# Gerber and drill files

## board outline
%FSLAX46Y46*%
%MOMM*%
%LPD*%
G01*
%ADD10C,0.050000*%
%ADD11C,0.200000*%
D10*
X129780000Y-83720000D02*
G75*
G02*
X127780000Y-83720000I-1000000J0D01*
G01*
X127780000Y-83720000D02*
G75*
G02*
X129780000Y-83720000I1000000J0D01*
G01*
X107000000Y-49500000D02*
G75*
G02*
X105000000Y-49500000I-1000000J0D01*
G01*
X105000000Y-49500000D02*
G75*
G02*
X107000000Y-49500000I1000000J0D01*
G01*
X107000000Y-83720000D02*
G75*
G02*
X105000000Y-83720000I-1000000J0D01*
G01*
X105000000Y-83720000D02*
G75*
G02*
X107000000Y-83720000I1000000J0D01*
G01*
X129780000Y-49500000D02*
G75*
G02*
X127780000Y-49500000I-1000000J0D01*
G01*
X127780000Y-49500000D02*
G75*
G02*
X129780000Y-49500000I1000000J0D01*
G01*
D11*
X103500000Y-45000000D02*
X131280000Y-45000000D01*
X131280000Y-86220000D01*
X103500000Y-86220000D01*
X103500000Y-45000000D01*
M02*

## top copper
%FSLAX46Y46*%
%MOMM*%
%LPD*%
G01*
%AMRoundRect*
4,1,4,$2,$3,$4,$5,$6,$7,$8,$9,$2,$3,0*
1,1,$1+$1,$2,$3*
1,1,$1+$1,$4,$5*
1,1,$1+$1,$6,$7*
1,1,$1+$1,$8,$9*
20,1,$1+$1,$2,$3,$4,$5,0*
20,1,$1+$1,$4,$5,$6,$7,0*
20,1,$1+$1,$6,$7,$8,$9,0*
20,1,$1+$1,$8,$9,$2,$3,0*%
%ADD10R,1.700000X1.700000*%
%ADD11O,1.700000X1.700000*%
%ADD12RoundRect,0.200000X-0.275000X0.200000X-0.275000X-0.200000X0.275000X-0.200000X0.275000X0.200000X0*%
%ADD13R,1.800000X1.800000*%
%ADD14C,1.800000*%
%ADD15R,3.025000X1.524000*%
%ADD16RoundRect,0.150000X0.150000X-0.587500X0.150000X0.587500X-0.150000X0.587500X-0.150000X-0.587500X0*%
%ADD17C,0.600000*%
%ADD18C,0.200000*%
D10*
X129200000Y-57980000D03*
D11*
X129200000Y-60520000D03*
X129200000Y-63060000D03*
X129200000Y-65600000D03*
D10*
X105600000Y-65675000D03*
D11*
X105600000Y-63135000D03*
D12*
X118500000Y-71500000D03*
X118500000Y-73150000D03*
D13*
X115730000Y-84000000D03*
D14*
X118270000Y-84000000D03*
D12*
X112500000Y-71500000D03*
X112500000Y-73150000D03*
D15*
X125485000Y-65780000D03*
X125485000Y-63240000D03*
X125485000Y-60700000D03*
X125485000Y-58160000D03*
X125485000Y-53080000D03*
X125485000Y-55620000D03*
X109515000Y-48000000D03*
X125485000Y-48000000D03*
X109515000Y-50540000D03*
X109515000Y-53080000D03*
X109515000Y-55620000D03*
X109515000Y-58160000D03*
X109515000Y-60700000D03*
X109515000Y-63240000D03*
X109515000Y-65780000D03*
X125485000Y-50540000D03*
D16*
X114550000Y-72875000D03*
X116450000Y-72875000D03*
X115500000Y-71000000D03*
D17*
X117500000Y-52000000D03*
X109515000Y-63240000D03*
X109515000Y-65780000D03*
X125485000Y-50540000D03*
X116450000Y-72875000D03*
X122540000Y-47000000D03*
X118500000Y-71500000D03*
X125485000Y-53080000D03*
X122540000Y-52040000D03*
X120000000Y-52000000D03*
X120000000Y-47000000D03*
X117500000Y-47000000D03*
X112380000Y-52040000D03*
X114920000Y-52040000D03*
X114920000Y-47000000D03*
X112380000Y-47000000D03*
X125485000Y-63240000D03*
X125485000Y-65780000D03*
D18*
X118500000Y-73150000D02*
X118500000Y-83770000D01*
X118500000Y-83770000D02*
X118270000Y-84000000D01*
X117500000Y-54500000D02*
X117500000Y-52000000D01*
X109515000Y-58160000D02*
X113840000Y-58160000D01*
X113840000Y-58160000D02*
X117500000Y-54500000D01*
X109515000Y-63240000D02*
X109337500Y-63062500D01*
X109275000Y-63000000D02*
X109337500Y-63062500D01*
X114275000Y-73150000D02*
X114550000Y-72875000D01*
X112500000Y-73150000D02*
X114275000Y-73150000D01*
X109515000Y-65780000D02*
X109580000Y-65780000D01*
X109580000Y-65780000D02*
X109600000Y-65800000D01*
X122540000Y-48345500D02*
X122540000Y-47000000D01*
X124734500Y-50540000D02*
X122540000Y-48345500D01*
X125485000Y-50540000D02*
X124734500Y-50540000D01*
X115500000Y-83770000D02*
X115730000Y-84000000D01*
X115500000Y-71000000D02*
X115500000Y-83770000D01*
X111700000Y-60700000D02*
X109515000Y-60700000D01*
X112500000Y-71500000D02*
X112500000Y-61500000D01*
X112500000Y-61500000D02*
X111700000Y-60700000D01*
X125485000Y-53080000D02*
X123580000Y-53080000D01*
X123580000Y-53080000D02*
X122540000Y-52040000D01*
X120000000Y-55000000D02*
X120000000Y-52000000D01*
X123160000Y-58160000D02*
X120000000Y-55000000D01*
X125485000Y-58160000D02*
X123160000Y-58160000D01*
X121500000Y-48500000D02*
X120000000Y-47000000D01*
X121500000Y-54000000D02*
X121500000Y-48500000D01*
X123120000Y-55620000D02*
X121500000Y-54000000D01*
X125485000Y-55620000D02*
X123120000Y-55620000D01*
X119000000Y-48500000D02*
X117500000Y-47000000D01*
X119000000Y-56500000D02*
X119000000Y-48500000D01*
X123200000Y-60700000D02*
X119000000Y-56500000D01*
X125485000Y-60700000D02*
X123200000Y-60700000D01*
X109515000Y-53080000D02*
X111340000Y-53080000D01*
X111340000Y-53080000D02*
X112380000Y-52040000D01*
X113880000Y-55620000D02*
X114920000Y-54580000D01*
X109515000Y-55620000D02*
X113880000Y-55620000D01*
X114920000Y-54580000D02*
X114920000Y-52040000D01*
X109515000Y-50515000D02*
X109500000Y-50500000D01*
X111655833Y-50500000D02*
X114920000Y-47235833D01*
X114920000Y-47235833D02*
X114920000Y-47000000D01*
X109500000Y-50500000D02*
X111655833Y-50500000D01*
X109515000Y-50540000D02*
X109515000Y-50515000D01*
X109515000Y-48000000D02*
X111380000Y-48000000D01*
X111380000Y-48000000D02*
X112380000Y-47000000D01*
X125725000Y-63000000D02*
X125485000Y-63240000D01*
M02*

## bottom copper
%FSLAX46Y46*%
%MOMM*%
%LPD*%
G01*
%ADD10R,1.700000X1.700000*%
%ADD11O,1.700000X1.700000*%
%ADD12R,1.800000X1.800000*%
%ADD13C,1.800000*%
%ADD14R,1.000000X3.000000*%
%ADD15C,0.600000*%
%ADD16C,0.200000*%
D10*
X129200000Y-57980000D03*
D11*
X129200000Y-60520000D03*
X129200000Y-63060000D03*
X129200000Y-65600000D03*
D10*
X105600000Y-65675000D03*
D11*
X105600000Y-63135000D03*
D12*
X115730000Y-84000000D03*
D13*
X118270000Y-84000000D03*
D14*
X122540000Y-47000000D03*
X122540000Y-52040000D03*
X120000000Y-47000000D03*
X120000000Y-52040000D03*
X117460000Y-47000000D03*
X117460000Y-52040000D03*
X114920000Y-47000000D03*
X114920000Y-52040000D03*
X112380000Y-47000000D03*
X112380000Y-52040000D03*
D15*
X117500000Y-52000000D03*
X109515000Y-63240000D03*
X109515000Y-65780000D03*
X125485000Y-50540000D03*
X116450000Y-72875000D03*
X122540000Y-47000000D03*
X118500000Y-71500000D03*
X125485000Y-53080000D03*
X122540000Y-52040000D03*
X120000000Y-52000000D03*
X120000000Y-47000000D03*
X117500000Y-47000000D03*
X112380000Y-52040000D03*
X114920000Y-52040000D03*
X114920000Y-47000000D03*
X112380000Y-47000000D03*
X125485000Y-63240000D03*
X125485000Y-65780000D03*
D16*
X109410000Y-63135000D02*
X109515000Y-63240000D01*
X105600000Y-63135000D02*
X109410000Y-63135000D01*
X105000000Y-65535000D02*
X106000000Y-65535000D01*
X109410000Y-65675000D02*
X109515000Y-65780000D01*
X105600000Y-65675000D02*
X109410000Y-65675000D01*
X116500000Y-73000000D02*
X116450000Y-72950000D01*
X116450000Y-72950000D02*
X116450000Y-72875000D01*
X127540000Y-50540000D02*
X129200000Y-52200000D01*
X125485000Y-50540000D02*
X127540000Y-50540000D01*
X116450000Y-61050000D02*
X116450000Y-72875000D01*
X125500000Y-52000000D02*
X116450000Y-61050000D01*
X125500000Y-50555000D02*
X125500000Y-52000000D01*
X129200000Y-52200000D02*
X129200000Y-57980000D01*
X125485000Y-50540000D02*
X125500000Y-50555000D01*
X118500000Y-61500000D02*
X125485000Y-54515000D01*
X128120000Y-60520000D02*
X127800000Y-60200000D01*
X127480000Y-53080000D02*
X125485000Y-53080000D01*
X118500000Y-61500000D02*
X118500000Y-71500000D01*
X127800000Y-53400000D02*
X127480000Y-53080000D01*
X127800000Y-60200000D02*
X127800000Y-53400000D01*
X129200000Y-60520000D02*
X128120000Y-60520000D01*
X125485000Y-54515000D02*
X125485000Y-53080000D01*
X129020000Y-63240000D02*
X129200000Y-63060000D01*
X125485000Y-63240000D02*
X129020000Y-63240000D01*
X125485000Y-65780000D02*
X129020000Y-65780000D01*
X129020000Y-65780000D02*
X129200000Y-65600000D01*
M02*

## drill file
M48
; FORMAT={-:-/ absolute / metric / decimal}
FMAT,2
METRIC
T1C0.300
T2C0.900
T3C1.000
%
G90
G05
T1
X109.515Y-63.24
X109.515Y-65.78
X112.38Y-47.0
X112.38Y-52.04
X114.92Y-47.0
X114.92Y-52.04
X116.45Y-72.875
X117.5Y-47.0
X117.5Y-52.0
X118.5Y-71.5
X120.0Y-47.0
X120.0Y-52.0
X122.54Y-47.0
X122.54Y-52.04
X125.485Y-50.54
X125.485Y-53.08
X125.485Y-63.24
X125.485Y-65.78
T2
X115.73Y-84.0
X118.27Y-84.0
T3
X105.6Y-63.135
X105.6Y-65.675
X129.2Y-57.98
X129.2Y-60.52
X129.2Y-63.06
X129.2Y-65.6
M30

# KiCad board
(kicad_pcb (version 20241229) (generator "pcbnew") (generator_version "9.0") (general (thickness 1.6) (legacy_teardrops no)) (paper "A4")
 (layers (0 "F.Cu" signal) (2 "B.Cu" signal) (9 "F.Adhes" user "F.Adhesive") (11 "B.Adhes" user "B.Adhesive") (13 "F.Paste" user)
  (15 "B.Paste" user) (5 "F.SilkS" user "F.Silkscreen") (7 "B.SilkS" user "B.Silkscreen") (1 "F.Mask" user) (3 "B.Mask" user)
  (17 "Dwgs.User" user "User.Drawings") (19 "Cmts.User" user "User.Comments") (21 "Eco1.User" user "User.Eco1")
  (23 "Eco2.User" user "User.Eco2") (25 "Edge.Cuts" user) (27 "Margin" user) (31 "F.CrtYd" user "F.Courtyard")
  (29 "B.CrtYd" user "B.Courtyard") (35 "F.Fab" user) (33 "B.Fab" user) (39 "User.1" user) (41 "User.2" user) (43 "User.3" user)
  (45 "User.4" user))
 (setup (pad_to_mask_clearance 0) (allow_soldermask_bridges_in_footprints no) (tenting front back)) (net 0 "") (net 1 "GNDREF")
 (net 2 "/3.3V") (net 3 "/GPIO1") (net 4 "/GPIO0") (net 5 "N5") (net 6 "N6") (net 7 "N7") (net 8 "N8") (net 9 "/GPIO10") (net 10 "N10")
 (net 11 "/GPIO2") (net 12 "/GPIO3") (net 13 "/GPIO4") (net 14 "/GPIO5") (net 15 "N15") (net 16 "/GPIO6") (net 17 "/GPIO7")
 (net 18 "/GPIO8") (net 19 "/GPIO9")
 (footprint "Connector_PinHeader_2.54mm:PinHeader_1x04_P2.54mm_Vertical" (layer "F.Cu") (at 129.2 57.98)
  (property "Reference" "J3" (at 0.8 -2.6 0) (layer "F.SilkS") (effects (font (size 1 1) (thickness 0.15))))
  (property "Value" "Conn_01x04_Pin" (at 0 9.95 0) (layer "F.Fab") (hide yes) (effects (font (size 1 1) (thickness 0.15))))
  (pad "1" thru_hole rect (at 0 0) (size 1.7 1.7) (drill 1) (layers "*.Cu" "*.Mask") (remove_unused_layers no) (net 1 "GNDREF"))
  (pad "2" thru_hole oval (at 0 2.54) (size 1.7 1.7) (drill 1) (layers "*.Cu" "*.Mask") (remove_unused_layers no) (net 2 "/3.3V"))
  (pad "3" thru_hole oval (at 0 5.08) (size 1.7 1.7) (drill 1) (layers "*.Cu" "*.Mask") (remove_unused_layers no) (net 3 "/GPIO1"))
  (pad "4" thru_hole oval (at 0 7.62) (size 1.7 1.7) (drill 1) (layers "*.Cu" "*.Mask") (remove_unused_layers no) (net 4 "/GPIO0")))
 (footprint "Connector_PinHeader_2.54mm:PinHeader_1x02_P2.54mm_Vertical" (layer "F.Cu") (at 105.6 65.675 180)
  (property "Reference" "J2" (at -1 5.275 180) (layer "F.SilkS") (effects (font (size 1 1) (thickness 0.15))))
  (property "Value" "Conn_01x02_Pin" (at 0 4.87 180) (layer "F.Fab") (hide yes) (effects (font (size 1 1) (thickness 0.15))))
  (pad "1" thru_hole rect (at 0 0 180) (size 1.7 1.7) (drill 1) (layers "*.Cu" "*.Mask") (remove_unused_layers no) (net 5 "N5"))
  (pad "2" thru_hole oval (at 0 2.54 180) (size 1.7 1.7) (drill 1) (layers "*.Cu" "*.Mask") (remove_unused_layers no) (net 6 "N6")))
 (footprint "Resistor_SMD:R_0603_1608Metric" (layer "F.Cu") (at 118.5 72.325 -90)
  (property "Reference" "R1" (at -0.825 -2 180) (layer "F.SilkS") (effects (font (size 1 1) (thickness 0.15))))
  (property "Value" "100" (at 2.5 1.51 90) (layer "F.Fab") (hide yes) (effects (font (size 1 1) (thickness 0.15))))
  (pad "1" smd roundrect (at -0.825 0 270) (size 0.8 0.95) (layers "F.Cu" "F.Mask" "F.Paste") (roundrect_rratio 0.25) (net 2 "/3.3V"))
  (pad "2" smd roundrect (at 0.825 0 270) (size 0.8 0.95) (layers "F.Cu" "F.Mask" "F.Paste") (roundrect_rratio 0.25) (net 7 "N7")))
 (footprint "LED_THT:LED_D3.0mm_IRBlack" (layer "F.Cu") (at 115.73 84)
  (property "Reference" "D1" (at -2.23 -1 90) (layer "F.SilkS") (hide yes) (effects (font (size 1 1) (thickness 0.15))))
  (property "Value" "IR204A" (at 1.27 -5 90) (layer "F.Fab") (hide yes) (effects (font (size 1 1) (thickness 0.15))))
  (pad "1" thru_hole rect (at 0 0) (size 1.8 1.8) (drill 0.9) (layers "*.Cu" "*.Mask") (remove_unused_layers no) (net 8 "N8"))
  (pad "2" thru_hole circle (at 2.54 0) (size 1.8 1.8) (drill 0.9) (layers "*.Cu" "*.Mask") (remove_unused_layers no) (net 7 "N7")))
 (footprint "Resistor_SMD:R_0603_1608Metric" (layer "F.Cu") (at 112.5 72.325 -90)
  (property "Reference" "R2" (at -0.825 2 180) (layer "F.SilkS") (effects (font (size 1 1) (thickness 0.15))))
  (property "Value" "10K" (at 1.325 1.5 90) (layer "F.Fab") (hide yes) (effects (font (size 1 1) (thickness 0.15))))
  (pad "1" smd roundrect (at -0.825 0 270) (size 0.8 0.95) (layers "F.Cu" "F.Mask" "F.Paste") (roundrect_rratio 0.25) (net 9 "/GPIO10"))
  (pad "2" smd roundrect (at 0.825 0 270) (size 0.8 0.95) (layers "F.Cu" "F.Mask" "F.Paste") (roundrect_rratio 0.25) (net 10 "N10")))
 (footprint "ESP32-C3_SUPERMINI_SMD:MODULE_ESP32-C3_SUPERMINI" (layer "F.Cu") (at 117.5 57.9)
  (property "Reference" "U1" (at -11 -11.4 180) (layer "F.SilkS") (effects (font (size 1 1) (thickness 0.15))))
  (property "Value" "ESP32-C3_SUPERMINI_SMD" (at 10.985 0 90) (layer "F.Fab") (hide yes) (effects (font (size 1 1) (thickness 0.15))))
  (pad "0" smd rect (at 7.985 7.88) (size 3.025 1.524) (layers "F.Cu" "F.Mask" "F.Paste") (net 4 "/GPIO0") (solder_mask_margin 0.102))
  (pad "1" smd rect (at 7.985 5.34) (size 3.025 1.524) (layers "F.Cu" "F.Mask" "F.Paste") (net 3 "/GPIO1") (solder_mask_margin 0.102))
  (pad "2" smd rect (at 7.985 2.8) (size 3.025 1.524) (layers "F.Cu" "F.Mask" "F.Paste") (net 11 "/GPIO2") (solder_mask_margin 0.102))
  (pad "3" smd rect (at 7.985 0.26) (size 3.025 1.524) (layers "F.Cu" "F.Mask" "F.Paste") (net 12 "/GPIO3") (solder_mask_margin 0.102))
  (pad "3.3" smd rect (at 7.985 -4.82) (size 3.025 1.524) (layers "F.Cu" "F.Mask" "F.Paste") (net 2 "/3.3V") (solder_mask_margin 0.102))
  (pad "4" smd rect (at 7.985 -2.28) (size 3.025 1.524) (layers "F.Cu" "F.Mask" "F.Paste") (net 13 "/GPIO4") (solder_mask_margin 0.102))
  (pad "5" smd rect (at -7.985 -9.9) (size 3.025 1.524) (layers "F.Cu" "F.Mask" "F.Paste") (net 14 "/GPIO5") (solder_mask_margin 0.102))
  (pad "5V" smd rect (at 7.985 -9.9) (size 3.025 1.524) (layers "F.Cu" "F.Mask" "F.Paste") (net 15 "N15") (solder_mask_margin 0.102))
  (pad "6" smd rect (at -7.985 -7.36) (size 3.025 1.524) (layers "F.Cu" "F.Mask" "F.Paste") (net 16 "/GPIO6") (solder_mask_margin 0.102))
  (pad "7" smd rect (at -7.985 -4.82) (size 3.025 1.524) (layers "F.Cu" "F.Mask" "F.Paste") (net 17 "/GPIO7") (solder_mask_margin 0.102))
  (pad "8" smd rect (at -7.985 -2.28) (size 3.025 1.524) (layers "F.Cu" "F.Mask" "F.Paste") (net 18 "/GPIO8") (solder_mask_margin 0.102))
  (pad "9" smd rect (at -7.985 0.26) (size 3.025 1.524) (layers "F.Cu" "F.Mask" "F.Paste") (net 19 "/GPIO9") (solder_mask_margin 0.102))
  (pad "10" smd rect (at -7.985 2.8) (size 3.025 1.524) (layers "F.Cu" "F.Mask" "F.Paste") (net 9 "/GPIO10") (solder_mask_margin 0.102))
  (pad "20" smd rect (at -7.985 5.34) (size 3.025 1.524) (layers "F.Cu" "F.Mask" "F.Paste") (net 6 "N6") (solder_mask_margin 0.102))
  (pad "21" smd rect (at -7.985 7.88) (size 3.025 1.524) (layers "F.Cu" "F.Mask" "F.Paste") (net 5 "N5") (solder_mask_margin 0.102))
  (pad "G" smd rect (at 7.985 -7.36) (size 3.025 1.524) (layers "F.Cu" "F.Mask" "F.Paste") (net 1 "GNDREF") (solder_mask_margin 0.102)))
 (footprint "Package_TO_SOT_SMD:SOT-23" (layer "F.Cu") (at 115.5 71.9375 90)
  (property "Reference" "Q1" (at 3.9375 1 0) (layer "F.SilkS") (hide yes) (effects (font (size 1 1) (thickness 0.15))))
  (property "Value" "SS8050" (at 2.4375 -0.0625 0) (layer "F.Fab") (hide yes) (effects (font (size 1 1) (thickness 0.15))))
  (pad "1" smd roundrect (at -0.9375 -0.95 90) (size 1.475 0.6) (layers "F.Cu" "F.Mask" "F.Paste") (roundrect_rratio 0.25) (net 10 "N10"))
  (pad "2" smd roundrect (at -0.9375 0.95 90) (size 1.475 0.6) (layers "F.Cu" "F.Mask" "F.Paste") (roundrect_rratio 0.25) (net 1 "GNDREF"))
  (pad "3" smd roundrect (at 0.9375 0 90) (size 1.475 0.6) (layers "F.Cu" "F.Mask" "F.Paste") (roundrect_rratio 0.25) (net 8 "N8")))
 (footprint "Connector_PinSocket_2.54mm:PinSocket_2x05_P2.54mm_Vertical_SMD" (layer "B.Cu") (at 117.46 49.52 90)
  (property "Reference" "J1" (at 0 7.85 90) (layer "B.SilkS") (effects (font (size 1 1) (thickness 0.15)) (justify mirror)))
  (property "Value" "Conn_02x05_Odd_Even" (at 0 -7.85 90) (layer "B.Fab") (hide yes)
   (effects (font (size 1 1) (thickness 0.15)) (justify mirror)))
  (pad "1" smd rect (at 2.52 5.08 90) (size 3 1) (layers "B.Cu" "B.Mask" "B.Paste") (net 1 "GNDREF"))
  (pad "2" smd rect (at -2.52 5.08 90) (size 3 1) (layers "B.Cu" "B.Mask" "B.Paste") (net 2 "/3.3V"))
  (pad "3" smd rect (at 2.52 2.54 90) (size 3 1) (layers "B.Cu" "B.Mask" "B.Paste") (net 13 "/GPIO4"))
  (pad "4" smd rect (at -2.52 2.54 90) (size 3 1) (layers "B.Cu" "B.Mask" "B.Paste") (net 12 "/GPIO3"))
  (pad "5" smd rect (at 2.52 0 90) (size 3 1) (layers "B.Cu" "B.Mask" "B.Paste") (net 11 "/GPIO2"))
  (pad "6" smd rect (at -2.52 0 90) (size 3 1) (layers "B.Cu" "B.Mask" "B.Paste") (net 19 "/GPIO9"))
  (pad "7" smd rect (at 2.52 -2.54 90) (size 3 1) (layers "B.Cu" "B.Mask" "B.Paste") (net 16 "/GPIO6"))
  (pad "8" smd rect (at -2.52 -2.54 90) (size 3 1) (layers "B.Cu" "B.Mask" "B.Paste") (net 18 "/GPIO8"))
  (pad "9" smd rect (at 2.52 -5.08 90) (size 3 1) (layers "B.Cu" "B.Mask" "B.Paste") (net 14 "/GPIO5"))
  (pad "10" smd rect (at -2.52 -5.08 90) (size 3 1) (layers "B.Cu" "B.Mask" "B.Paste") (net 17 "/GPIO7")))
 (gr_circle (center 128.78 83.72) (end 129.78 83.72) (stroke (width 0.05) (type solid)) (fill no) (layer "Edge.Cuts"))
 (gr_circle (center 106 49.5) (end 107 49.5) (stroke (width 0.05) (type solid)) (fill no) (layer "Edge.Cuts"))
 (gr_circle (center 106 83.72) (end 107 83.72) (stroke (width 0.05) (type solid)) (fill no) (layer "Edge.Cuts"))
 (gr_circle (center 128.78 49.5) (end 129.78 49.5) (stroke (width 0.05) (type solid)) (fill no) (layer "Edge.Cuts"))
 (gr_rect (start 103.5 45) (end 131.28 86.22) (stroke (width 0.2) (type solid)) (fill no) (layer "Edge.Cuts"))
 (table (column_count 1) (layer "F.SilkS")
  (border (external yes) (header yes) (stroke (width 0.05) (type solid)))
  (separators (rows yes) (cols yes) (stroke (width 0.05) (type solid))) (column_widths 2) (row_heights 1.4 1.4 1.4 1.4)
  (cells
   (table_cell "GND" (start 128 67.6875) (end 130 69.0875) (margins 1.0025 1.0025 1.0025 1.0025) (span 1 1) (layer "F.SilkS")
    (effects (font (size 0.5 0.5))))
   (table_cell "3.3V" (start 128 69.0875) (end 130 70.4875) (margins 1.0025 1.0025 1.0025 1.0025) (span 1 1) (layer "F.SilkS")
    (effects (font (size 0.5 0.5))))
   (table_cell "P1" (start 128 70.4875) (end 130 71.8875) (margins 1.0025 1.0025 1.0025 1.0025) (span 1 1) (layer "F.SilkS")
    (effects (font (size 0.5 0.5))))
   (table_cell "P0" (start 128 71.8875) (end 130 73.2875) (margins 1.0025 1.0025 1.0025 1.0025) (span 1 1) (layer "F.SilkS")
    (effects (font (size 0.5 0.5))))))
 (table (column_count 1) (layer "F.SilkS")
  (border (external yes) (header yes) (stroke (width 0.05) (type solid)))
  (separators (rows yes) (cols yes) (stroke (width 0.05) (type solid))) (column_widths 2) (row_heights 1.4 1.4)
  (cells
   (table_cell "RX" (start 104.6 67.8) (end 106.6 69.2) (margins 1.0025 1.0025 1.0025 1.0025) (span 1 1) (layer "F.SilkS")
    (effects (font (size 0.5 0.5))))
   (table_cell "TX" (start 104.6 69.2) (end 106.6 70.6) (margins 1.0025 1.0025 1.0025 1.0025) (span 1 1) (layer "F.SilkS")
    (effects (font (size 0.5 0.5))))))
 (segment (start 118.5 73.15) (end 118.5 83.77) (width 0.2) (layer "F.Cu") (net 7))
 (segment (start 118.5 83.77) (end 118.27 84) (width 0.2) (layer "F.Cu") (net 7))
 (segment (start 117.5 54.5) (end 117.5 52) (width 0.2) (layer "F.Cu") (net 19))
 (segment (start 109.515 58.16) (end 113.84 58.16) (width 0.2) (layer "F.Cu") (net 19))
 (segment (start 113.84 58.16) (end 117.5 54.5) (width 0.2) (layer "F.Cu") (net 19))
 (via (at 117.5 52) (size 0.6) (drill 0.3) (layers "F.Cu" "B.Cu") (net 19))
 (segment (start 109.515 63.24) (end 109.3375 63.0625) (width 0.2) (layer "F.Cu") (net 6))
 (segment (start 109.275 63) (end 109.3375 63.0625) (width 0.2) (layer "F.Cu") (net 6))
 (via (at 109.515 63.24) (size 0.6) (drill 0.3) (layers "F.Cu" "B.Cu") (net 6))
 (segment (start 109.41 63.135) (end 109.515 63.24) (width 0.2) (layer "B.Cu") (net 6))
 (segment (start 105.6 63.135) (end 109.41 63.135) (width 0.2) (layer "B.Cu") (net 6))
 (segment (start 114.275 73.15) (end 114.55 72.875) (width 0.2) (layer "F.Cu") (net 10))
 (segment (start 112.5 73.15) (end 114.275 73.15) (width 0.2) (layer "F.Cu") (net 10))
 (segment (start 109.515 65.78) (end 109.58 65.78) (width 0.2) (layer "F.Cu") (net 5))
 (segment (start 109.58 65.78) (end 109.6 65.8) (width 0.2) (layer "F.Cu") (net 5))
 (via (at 109.515 65.78) (size 0.6) (drill 0.3) (layers "F.Cu" "B.Cu") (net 5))
 (segment (start 105 65.535) (end 106 65.535) (width 0.2) (layer "B.Cu") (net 5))
 (segment (start 109.41 65.675) (end 109.515 65.78) (width 0.2) (layer "B.Cu") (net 5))
 (segment (start 105.6 65.675) (end 109.41 65.675) (width 0.2) (layer "B.Cu") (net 5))
 (segment (start 122.54 48.3455) (end 122.54 47) (width 0.2) (layer "F.Cu") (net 1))
 (segment (start 124.7345 50.54) (end 122.54 48.3455) (width 0.2) (layer "F.Cu") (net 1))
 (segment (start 125.485 50.54) (end 124.7345 50.54) (width 0.2) (layer "F.Cu") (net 1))
 (via (at 125.485 50.54) (size 0.6) (drill 0.3) (layers "F.Cu" "B.Cu") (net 1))
 (via (at 116.45 72.875) (size 0.6) (drill 0.3) (layers "F.Cu" "B.Cu") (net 1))
 (via (at 122.54 47) (size 0.6) (drill 0.3) (layers "F.Cu" "B.Cu") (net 1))
 (segment (start 116.5 73) (end 116.45 72.95) (width 0.2) (layer "B.Cu") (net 1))
 (segment (start 116.45 72.95) (end 116.45 72.875) (width 0.2) (layer "B.Cu") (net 1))
 (segment (start 127.54 50.54) (end 129.2 52.2) (width 0.2) (layer "B.Cu") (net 1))
 (segment (start 125.485 50.54) (end 127.54 50.54) (width 0.2) (layer "B.Cu") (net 1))
 (segment (start 116.45 61.05) (end 116.45 72.875) (width 0.2) (layer "B.Cu") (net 1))
 (segment (start 125.5 52) (end 116.45 61.05) (width 0.2) (layer "B.Cu") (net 1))
 (segment (start 125.5 50.555) (end 125.5 52) (width 0.2) (layer "B.Cu") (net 1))
 (segment (start 129.2 52.2) (end 129.2 57.98) (width 0.2) (layer "B.Cu") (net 1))
 (segment (start 125.485 50.54) (end 125.5 50.555) (width 0.2) (layer "B.Cu") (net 1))
 (segment (start 115.5 83.77) (end 115.73 84) (width 0.2) (layer "F.Cu") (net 8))
 (segment (start 115.5 71) (end 115.5 83.77) (width 0.2) (layer "F.Cu") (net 8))
 (segment (start 111.7 60.7) (end 109.515 60.7) (width 0.2) (layer "F.Cu") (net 9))
 (segment (start 112.5 71.5) (end 112.5 61.5) (width 0.2) (layer "F.Cu") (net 9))
 (segment (start 112.5 61.5) (end 111.7 60.7) (width 0.2) (layer "F.Cu") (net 9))
 (segment (start 125.485 53.08) (end 123.58 53.08) (width 0.2) (layer "F.Cu") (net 2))
 (segment (start 123.58 53.08) (end 122.54 52.04) (width 0.2) (layer "F.Cu") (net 2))
 (via (at 118.5 71.5) (size 0.6) (drill 0.3) (layers "F.Cu" "B.Cu") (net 2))
 (via (at 125.485 53.08) (size 0.6) (drill 0.3) (layers "F.Cu" "B.Cu") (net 2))
 (via (at 122.54 52.04) (size 0.6) (drill 0.3) (layers "F.Cu" "B.Cu") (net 2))
 (segment (start 118.5 61.5) (end 125.485 54.515) (width 0.2) (layer "B.Cu") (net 2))
 (segment (start 128.12 60.52) (end 127.8 60.2) (width 0.2) (layer "B.Cu") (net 2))
 (segment (start 127.48 53.08) (end 125.485 53.08) (width 0.2) (layer "B.Cu") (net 2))
 (segment (start 118.5 61.5) (end 118.5 71.5) (width 0.2) (layer "B.Cu") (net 2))
 (segment (start 127.8 53.4) (end 127.48 53.08) (width 0.2) (layer "B.Cu") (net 2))
 (segment (start 127.8 60.2) (end 127.8 53.4) (width 0.2) (layer "B.Cu") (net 2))
 (segment (start 129.2 60.52) (end 128.12 60.52) (width 0.2) (layer "B.Cu") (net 2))
 (segment (start 125.485 54.515) (end 125.485 53.08) (width 0.2) (layer "B.Cu") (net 2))
 (segment (start 120 55) (end 120 52) (width 0.2) (layer "F.Cu") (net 12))
 (segment (start 123.16 58.16) (end 120 55) (width 0.2) (layer "F.Cu") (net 12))
 (segment (start 125.485 58.16) (end 123.16 58.16) (width 0.2) (layer "F.Cu") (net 12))
 (via (at 120 52) (size 0.6) (drill 0.3) (layers "F.Cu" "B.Cu") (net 12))
 (segment (start 121.5 48.5) (end 120 47) (width 0.2) (layer "F.Cu") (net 13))
 (segment (start 121.5 54) (end 121.5 48.5) (width 0.2) (layer "F.Cu") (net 13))
 (segment (start 123.12 55.62) (end 121.5 54) (width 0.2) (layer "F.Cu") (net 13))
 (segment (start 125.485 55.62) (end 123.12 55.62) (width 0.2) (layer "F.Cu") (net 13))
 (via (at 120 47) (size 0.6) (drill 0.3) (layers "F.Cu" "B.Cu") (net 13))
 (segment (start 119 48.5) (end 117.5 47) (width 0.2) (layer "F.Cu") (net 11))
 (segment (start 119 56.5) (end 119 48.5) (width 0.2) (layer "F.Cu") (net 11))
 (segment (start 123.2 60.7) (end 119 56.5) (width 0.2) (layer "F.Cu") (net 11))
 (segment (start 125.485 60.7) (end 123.2 60.7) (width 0.2) (layer "F.Cu") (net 11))
 (via (at 117.5 47) (size 0.6) (drill 0.3) (layers "F.Cu" "B.Cu") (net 11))
 (segment (start 109.515 53.08) (end 111.34 53.08) (width 0.2) (layer "F.Cu") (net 17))
 (segment (start 111.34 53.08) (end 112.38 52.04) (width 0.2) (layer "F.Cu") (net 17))
 (via (at 112.38 52.04) (size 0.6) (drill 0.3) (layers "F.Cu" "B.Cu") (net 17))
 (segment (start 113.88 55.62) (end 114.92 54.58) (width 0.2) (layer "F.Cu") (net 18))
 (segment (start 109.515 55.62) (end 113.88 55.62) (width 0.2) (layer "F.Cu") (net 18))
 (segment (start 114.92 54.58) (end 114.92 52.04) (width 0.2) (layer "F.Cu") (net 18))
 (via (at 114.92 52.04) (size 0.6) (drill 0.3) (layers "F.Cu" "B.Cu") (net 18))
 (segment (start 109.515 50.515) (end 109.5 50.5) (width 0.2) (layer "F.Cu") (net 16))
 (segment (start 111.655833 50.5) (end 114.92 47.235833) (width 0.2) (layer "F.Cu") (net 16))
 (segment (start 114.92 47.235833) (end 114.92 47) (width 0.2) (layer "F.Cu") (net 16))
 (segment (start 109.5 50.5) (end 111.655833 50.5) (width 0.2) (layer "F.Cu") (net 16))
 (segment (start 109.515 50.54) (end 109.515 50.515) (width 0.2) (layer "F.Cu") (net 16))
 (via (at 114.92 47) (size 0.6) (drill 0.3) (layers "F.Cu" "B.Cu") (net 16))
 (segment (start 109.515 48) (end 111.38 48) (width 0.2) (layer "F.Cu") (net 14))
 (segment (start 111.38 48) (end 112.38 47) (width 0.2) (layer "F.Cu") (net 14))
 (via (at 112.38 47) (size 0.6) (drill 0.3) (layers "F.Cu" "B.Cu") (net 14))
 (segment (start 125.725 63) (end 125.485 63.24) (width 0.2) (layer "F.Cu") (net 3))
 (via (at 125.485 63.24) (size 0.6) (drill 0.3) (layers "F.Cu" "B.Cu") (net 3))
 (segment (start 129.02 63.24) (end 129.2 63.06) (width 0.2) (layer "B.Cu") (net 3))
 (segment (start 125.485 63.24) (end 129.02 63.24) (width 0.2) (layer "B.Cu") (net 3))
 (via (at 125.485 65.78) (size 0.6) (drill 0.3) (layers "F.Cu" "B.Cu") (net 4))
 (segment (start 125.485 65.78) (end 129.02 65.78) (width 0.2) (layer "B.Cu") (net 4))
 (segment (start 129.02 65.78) (end 129.2 65.6) (width 0.2) (layer "B.Cu") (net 4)))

